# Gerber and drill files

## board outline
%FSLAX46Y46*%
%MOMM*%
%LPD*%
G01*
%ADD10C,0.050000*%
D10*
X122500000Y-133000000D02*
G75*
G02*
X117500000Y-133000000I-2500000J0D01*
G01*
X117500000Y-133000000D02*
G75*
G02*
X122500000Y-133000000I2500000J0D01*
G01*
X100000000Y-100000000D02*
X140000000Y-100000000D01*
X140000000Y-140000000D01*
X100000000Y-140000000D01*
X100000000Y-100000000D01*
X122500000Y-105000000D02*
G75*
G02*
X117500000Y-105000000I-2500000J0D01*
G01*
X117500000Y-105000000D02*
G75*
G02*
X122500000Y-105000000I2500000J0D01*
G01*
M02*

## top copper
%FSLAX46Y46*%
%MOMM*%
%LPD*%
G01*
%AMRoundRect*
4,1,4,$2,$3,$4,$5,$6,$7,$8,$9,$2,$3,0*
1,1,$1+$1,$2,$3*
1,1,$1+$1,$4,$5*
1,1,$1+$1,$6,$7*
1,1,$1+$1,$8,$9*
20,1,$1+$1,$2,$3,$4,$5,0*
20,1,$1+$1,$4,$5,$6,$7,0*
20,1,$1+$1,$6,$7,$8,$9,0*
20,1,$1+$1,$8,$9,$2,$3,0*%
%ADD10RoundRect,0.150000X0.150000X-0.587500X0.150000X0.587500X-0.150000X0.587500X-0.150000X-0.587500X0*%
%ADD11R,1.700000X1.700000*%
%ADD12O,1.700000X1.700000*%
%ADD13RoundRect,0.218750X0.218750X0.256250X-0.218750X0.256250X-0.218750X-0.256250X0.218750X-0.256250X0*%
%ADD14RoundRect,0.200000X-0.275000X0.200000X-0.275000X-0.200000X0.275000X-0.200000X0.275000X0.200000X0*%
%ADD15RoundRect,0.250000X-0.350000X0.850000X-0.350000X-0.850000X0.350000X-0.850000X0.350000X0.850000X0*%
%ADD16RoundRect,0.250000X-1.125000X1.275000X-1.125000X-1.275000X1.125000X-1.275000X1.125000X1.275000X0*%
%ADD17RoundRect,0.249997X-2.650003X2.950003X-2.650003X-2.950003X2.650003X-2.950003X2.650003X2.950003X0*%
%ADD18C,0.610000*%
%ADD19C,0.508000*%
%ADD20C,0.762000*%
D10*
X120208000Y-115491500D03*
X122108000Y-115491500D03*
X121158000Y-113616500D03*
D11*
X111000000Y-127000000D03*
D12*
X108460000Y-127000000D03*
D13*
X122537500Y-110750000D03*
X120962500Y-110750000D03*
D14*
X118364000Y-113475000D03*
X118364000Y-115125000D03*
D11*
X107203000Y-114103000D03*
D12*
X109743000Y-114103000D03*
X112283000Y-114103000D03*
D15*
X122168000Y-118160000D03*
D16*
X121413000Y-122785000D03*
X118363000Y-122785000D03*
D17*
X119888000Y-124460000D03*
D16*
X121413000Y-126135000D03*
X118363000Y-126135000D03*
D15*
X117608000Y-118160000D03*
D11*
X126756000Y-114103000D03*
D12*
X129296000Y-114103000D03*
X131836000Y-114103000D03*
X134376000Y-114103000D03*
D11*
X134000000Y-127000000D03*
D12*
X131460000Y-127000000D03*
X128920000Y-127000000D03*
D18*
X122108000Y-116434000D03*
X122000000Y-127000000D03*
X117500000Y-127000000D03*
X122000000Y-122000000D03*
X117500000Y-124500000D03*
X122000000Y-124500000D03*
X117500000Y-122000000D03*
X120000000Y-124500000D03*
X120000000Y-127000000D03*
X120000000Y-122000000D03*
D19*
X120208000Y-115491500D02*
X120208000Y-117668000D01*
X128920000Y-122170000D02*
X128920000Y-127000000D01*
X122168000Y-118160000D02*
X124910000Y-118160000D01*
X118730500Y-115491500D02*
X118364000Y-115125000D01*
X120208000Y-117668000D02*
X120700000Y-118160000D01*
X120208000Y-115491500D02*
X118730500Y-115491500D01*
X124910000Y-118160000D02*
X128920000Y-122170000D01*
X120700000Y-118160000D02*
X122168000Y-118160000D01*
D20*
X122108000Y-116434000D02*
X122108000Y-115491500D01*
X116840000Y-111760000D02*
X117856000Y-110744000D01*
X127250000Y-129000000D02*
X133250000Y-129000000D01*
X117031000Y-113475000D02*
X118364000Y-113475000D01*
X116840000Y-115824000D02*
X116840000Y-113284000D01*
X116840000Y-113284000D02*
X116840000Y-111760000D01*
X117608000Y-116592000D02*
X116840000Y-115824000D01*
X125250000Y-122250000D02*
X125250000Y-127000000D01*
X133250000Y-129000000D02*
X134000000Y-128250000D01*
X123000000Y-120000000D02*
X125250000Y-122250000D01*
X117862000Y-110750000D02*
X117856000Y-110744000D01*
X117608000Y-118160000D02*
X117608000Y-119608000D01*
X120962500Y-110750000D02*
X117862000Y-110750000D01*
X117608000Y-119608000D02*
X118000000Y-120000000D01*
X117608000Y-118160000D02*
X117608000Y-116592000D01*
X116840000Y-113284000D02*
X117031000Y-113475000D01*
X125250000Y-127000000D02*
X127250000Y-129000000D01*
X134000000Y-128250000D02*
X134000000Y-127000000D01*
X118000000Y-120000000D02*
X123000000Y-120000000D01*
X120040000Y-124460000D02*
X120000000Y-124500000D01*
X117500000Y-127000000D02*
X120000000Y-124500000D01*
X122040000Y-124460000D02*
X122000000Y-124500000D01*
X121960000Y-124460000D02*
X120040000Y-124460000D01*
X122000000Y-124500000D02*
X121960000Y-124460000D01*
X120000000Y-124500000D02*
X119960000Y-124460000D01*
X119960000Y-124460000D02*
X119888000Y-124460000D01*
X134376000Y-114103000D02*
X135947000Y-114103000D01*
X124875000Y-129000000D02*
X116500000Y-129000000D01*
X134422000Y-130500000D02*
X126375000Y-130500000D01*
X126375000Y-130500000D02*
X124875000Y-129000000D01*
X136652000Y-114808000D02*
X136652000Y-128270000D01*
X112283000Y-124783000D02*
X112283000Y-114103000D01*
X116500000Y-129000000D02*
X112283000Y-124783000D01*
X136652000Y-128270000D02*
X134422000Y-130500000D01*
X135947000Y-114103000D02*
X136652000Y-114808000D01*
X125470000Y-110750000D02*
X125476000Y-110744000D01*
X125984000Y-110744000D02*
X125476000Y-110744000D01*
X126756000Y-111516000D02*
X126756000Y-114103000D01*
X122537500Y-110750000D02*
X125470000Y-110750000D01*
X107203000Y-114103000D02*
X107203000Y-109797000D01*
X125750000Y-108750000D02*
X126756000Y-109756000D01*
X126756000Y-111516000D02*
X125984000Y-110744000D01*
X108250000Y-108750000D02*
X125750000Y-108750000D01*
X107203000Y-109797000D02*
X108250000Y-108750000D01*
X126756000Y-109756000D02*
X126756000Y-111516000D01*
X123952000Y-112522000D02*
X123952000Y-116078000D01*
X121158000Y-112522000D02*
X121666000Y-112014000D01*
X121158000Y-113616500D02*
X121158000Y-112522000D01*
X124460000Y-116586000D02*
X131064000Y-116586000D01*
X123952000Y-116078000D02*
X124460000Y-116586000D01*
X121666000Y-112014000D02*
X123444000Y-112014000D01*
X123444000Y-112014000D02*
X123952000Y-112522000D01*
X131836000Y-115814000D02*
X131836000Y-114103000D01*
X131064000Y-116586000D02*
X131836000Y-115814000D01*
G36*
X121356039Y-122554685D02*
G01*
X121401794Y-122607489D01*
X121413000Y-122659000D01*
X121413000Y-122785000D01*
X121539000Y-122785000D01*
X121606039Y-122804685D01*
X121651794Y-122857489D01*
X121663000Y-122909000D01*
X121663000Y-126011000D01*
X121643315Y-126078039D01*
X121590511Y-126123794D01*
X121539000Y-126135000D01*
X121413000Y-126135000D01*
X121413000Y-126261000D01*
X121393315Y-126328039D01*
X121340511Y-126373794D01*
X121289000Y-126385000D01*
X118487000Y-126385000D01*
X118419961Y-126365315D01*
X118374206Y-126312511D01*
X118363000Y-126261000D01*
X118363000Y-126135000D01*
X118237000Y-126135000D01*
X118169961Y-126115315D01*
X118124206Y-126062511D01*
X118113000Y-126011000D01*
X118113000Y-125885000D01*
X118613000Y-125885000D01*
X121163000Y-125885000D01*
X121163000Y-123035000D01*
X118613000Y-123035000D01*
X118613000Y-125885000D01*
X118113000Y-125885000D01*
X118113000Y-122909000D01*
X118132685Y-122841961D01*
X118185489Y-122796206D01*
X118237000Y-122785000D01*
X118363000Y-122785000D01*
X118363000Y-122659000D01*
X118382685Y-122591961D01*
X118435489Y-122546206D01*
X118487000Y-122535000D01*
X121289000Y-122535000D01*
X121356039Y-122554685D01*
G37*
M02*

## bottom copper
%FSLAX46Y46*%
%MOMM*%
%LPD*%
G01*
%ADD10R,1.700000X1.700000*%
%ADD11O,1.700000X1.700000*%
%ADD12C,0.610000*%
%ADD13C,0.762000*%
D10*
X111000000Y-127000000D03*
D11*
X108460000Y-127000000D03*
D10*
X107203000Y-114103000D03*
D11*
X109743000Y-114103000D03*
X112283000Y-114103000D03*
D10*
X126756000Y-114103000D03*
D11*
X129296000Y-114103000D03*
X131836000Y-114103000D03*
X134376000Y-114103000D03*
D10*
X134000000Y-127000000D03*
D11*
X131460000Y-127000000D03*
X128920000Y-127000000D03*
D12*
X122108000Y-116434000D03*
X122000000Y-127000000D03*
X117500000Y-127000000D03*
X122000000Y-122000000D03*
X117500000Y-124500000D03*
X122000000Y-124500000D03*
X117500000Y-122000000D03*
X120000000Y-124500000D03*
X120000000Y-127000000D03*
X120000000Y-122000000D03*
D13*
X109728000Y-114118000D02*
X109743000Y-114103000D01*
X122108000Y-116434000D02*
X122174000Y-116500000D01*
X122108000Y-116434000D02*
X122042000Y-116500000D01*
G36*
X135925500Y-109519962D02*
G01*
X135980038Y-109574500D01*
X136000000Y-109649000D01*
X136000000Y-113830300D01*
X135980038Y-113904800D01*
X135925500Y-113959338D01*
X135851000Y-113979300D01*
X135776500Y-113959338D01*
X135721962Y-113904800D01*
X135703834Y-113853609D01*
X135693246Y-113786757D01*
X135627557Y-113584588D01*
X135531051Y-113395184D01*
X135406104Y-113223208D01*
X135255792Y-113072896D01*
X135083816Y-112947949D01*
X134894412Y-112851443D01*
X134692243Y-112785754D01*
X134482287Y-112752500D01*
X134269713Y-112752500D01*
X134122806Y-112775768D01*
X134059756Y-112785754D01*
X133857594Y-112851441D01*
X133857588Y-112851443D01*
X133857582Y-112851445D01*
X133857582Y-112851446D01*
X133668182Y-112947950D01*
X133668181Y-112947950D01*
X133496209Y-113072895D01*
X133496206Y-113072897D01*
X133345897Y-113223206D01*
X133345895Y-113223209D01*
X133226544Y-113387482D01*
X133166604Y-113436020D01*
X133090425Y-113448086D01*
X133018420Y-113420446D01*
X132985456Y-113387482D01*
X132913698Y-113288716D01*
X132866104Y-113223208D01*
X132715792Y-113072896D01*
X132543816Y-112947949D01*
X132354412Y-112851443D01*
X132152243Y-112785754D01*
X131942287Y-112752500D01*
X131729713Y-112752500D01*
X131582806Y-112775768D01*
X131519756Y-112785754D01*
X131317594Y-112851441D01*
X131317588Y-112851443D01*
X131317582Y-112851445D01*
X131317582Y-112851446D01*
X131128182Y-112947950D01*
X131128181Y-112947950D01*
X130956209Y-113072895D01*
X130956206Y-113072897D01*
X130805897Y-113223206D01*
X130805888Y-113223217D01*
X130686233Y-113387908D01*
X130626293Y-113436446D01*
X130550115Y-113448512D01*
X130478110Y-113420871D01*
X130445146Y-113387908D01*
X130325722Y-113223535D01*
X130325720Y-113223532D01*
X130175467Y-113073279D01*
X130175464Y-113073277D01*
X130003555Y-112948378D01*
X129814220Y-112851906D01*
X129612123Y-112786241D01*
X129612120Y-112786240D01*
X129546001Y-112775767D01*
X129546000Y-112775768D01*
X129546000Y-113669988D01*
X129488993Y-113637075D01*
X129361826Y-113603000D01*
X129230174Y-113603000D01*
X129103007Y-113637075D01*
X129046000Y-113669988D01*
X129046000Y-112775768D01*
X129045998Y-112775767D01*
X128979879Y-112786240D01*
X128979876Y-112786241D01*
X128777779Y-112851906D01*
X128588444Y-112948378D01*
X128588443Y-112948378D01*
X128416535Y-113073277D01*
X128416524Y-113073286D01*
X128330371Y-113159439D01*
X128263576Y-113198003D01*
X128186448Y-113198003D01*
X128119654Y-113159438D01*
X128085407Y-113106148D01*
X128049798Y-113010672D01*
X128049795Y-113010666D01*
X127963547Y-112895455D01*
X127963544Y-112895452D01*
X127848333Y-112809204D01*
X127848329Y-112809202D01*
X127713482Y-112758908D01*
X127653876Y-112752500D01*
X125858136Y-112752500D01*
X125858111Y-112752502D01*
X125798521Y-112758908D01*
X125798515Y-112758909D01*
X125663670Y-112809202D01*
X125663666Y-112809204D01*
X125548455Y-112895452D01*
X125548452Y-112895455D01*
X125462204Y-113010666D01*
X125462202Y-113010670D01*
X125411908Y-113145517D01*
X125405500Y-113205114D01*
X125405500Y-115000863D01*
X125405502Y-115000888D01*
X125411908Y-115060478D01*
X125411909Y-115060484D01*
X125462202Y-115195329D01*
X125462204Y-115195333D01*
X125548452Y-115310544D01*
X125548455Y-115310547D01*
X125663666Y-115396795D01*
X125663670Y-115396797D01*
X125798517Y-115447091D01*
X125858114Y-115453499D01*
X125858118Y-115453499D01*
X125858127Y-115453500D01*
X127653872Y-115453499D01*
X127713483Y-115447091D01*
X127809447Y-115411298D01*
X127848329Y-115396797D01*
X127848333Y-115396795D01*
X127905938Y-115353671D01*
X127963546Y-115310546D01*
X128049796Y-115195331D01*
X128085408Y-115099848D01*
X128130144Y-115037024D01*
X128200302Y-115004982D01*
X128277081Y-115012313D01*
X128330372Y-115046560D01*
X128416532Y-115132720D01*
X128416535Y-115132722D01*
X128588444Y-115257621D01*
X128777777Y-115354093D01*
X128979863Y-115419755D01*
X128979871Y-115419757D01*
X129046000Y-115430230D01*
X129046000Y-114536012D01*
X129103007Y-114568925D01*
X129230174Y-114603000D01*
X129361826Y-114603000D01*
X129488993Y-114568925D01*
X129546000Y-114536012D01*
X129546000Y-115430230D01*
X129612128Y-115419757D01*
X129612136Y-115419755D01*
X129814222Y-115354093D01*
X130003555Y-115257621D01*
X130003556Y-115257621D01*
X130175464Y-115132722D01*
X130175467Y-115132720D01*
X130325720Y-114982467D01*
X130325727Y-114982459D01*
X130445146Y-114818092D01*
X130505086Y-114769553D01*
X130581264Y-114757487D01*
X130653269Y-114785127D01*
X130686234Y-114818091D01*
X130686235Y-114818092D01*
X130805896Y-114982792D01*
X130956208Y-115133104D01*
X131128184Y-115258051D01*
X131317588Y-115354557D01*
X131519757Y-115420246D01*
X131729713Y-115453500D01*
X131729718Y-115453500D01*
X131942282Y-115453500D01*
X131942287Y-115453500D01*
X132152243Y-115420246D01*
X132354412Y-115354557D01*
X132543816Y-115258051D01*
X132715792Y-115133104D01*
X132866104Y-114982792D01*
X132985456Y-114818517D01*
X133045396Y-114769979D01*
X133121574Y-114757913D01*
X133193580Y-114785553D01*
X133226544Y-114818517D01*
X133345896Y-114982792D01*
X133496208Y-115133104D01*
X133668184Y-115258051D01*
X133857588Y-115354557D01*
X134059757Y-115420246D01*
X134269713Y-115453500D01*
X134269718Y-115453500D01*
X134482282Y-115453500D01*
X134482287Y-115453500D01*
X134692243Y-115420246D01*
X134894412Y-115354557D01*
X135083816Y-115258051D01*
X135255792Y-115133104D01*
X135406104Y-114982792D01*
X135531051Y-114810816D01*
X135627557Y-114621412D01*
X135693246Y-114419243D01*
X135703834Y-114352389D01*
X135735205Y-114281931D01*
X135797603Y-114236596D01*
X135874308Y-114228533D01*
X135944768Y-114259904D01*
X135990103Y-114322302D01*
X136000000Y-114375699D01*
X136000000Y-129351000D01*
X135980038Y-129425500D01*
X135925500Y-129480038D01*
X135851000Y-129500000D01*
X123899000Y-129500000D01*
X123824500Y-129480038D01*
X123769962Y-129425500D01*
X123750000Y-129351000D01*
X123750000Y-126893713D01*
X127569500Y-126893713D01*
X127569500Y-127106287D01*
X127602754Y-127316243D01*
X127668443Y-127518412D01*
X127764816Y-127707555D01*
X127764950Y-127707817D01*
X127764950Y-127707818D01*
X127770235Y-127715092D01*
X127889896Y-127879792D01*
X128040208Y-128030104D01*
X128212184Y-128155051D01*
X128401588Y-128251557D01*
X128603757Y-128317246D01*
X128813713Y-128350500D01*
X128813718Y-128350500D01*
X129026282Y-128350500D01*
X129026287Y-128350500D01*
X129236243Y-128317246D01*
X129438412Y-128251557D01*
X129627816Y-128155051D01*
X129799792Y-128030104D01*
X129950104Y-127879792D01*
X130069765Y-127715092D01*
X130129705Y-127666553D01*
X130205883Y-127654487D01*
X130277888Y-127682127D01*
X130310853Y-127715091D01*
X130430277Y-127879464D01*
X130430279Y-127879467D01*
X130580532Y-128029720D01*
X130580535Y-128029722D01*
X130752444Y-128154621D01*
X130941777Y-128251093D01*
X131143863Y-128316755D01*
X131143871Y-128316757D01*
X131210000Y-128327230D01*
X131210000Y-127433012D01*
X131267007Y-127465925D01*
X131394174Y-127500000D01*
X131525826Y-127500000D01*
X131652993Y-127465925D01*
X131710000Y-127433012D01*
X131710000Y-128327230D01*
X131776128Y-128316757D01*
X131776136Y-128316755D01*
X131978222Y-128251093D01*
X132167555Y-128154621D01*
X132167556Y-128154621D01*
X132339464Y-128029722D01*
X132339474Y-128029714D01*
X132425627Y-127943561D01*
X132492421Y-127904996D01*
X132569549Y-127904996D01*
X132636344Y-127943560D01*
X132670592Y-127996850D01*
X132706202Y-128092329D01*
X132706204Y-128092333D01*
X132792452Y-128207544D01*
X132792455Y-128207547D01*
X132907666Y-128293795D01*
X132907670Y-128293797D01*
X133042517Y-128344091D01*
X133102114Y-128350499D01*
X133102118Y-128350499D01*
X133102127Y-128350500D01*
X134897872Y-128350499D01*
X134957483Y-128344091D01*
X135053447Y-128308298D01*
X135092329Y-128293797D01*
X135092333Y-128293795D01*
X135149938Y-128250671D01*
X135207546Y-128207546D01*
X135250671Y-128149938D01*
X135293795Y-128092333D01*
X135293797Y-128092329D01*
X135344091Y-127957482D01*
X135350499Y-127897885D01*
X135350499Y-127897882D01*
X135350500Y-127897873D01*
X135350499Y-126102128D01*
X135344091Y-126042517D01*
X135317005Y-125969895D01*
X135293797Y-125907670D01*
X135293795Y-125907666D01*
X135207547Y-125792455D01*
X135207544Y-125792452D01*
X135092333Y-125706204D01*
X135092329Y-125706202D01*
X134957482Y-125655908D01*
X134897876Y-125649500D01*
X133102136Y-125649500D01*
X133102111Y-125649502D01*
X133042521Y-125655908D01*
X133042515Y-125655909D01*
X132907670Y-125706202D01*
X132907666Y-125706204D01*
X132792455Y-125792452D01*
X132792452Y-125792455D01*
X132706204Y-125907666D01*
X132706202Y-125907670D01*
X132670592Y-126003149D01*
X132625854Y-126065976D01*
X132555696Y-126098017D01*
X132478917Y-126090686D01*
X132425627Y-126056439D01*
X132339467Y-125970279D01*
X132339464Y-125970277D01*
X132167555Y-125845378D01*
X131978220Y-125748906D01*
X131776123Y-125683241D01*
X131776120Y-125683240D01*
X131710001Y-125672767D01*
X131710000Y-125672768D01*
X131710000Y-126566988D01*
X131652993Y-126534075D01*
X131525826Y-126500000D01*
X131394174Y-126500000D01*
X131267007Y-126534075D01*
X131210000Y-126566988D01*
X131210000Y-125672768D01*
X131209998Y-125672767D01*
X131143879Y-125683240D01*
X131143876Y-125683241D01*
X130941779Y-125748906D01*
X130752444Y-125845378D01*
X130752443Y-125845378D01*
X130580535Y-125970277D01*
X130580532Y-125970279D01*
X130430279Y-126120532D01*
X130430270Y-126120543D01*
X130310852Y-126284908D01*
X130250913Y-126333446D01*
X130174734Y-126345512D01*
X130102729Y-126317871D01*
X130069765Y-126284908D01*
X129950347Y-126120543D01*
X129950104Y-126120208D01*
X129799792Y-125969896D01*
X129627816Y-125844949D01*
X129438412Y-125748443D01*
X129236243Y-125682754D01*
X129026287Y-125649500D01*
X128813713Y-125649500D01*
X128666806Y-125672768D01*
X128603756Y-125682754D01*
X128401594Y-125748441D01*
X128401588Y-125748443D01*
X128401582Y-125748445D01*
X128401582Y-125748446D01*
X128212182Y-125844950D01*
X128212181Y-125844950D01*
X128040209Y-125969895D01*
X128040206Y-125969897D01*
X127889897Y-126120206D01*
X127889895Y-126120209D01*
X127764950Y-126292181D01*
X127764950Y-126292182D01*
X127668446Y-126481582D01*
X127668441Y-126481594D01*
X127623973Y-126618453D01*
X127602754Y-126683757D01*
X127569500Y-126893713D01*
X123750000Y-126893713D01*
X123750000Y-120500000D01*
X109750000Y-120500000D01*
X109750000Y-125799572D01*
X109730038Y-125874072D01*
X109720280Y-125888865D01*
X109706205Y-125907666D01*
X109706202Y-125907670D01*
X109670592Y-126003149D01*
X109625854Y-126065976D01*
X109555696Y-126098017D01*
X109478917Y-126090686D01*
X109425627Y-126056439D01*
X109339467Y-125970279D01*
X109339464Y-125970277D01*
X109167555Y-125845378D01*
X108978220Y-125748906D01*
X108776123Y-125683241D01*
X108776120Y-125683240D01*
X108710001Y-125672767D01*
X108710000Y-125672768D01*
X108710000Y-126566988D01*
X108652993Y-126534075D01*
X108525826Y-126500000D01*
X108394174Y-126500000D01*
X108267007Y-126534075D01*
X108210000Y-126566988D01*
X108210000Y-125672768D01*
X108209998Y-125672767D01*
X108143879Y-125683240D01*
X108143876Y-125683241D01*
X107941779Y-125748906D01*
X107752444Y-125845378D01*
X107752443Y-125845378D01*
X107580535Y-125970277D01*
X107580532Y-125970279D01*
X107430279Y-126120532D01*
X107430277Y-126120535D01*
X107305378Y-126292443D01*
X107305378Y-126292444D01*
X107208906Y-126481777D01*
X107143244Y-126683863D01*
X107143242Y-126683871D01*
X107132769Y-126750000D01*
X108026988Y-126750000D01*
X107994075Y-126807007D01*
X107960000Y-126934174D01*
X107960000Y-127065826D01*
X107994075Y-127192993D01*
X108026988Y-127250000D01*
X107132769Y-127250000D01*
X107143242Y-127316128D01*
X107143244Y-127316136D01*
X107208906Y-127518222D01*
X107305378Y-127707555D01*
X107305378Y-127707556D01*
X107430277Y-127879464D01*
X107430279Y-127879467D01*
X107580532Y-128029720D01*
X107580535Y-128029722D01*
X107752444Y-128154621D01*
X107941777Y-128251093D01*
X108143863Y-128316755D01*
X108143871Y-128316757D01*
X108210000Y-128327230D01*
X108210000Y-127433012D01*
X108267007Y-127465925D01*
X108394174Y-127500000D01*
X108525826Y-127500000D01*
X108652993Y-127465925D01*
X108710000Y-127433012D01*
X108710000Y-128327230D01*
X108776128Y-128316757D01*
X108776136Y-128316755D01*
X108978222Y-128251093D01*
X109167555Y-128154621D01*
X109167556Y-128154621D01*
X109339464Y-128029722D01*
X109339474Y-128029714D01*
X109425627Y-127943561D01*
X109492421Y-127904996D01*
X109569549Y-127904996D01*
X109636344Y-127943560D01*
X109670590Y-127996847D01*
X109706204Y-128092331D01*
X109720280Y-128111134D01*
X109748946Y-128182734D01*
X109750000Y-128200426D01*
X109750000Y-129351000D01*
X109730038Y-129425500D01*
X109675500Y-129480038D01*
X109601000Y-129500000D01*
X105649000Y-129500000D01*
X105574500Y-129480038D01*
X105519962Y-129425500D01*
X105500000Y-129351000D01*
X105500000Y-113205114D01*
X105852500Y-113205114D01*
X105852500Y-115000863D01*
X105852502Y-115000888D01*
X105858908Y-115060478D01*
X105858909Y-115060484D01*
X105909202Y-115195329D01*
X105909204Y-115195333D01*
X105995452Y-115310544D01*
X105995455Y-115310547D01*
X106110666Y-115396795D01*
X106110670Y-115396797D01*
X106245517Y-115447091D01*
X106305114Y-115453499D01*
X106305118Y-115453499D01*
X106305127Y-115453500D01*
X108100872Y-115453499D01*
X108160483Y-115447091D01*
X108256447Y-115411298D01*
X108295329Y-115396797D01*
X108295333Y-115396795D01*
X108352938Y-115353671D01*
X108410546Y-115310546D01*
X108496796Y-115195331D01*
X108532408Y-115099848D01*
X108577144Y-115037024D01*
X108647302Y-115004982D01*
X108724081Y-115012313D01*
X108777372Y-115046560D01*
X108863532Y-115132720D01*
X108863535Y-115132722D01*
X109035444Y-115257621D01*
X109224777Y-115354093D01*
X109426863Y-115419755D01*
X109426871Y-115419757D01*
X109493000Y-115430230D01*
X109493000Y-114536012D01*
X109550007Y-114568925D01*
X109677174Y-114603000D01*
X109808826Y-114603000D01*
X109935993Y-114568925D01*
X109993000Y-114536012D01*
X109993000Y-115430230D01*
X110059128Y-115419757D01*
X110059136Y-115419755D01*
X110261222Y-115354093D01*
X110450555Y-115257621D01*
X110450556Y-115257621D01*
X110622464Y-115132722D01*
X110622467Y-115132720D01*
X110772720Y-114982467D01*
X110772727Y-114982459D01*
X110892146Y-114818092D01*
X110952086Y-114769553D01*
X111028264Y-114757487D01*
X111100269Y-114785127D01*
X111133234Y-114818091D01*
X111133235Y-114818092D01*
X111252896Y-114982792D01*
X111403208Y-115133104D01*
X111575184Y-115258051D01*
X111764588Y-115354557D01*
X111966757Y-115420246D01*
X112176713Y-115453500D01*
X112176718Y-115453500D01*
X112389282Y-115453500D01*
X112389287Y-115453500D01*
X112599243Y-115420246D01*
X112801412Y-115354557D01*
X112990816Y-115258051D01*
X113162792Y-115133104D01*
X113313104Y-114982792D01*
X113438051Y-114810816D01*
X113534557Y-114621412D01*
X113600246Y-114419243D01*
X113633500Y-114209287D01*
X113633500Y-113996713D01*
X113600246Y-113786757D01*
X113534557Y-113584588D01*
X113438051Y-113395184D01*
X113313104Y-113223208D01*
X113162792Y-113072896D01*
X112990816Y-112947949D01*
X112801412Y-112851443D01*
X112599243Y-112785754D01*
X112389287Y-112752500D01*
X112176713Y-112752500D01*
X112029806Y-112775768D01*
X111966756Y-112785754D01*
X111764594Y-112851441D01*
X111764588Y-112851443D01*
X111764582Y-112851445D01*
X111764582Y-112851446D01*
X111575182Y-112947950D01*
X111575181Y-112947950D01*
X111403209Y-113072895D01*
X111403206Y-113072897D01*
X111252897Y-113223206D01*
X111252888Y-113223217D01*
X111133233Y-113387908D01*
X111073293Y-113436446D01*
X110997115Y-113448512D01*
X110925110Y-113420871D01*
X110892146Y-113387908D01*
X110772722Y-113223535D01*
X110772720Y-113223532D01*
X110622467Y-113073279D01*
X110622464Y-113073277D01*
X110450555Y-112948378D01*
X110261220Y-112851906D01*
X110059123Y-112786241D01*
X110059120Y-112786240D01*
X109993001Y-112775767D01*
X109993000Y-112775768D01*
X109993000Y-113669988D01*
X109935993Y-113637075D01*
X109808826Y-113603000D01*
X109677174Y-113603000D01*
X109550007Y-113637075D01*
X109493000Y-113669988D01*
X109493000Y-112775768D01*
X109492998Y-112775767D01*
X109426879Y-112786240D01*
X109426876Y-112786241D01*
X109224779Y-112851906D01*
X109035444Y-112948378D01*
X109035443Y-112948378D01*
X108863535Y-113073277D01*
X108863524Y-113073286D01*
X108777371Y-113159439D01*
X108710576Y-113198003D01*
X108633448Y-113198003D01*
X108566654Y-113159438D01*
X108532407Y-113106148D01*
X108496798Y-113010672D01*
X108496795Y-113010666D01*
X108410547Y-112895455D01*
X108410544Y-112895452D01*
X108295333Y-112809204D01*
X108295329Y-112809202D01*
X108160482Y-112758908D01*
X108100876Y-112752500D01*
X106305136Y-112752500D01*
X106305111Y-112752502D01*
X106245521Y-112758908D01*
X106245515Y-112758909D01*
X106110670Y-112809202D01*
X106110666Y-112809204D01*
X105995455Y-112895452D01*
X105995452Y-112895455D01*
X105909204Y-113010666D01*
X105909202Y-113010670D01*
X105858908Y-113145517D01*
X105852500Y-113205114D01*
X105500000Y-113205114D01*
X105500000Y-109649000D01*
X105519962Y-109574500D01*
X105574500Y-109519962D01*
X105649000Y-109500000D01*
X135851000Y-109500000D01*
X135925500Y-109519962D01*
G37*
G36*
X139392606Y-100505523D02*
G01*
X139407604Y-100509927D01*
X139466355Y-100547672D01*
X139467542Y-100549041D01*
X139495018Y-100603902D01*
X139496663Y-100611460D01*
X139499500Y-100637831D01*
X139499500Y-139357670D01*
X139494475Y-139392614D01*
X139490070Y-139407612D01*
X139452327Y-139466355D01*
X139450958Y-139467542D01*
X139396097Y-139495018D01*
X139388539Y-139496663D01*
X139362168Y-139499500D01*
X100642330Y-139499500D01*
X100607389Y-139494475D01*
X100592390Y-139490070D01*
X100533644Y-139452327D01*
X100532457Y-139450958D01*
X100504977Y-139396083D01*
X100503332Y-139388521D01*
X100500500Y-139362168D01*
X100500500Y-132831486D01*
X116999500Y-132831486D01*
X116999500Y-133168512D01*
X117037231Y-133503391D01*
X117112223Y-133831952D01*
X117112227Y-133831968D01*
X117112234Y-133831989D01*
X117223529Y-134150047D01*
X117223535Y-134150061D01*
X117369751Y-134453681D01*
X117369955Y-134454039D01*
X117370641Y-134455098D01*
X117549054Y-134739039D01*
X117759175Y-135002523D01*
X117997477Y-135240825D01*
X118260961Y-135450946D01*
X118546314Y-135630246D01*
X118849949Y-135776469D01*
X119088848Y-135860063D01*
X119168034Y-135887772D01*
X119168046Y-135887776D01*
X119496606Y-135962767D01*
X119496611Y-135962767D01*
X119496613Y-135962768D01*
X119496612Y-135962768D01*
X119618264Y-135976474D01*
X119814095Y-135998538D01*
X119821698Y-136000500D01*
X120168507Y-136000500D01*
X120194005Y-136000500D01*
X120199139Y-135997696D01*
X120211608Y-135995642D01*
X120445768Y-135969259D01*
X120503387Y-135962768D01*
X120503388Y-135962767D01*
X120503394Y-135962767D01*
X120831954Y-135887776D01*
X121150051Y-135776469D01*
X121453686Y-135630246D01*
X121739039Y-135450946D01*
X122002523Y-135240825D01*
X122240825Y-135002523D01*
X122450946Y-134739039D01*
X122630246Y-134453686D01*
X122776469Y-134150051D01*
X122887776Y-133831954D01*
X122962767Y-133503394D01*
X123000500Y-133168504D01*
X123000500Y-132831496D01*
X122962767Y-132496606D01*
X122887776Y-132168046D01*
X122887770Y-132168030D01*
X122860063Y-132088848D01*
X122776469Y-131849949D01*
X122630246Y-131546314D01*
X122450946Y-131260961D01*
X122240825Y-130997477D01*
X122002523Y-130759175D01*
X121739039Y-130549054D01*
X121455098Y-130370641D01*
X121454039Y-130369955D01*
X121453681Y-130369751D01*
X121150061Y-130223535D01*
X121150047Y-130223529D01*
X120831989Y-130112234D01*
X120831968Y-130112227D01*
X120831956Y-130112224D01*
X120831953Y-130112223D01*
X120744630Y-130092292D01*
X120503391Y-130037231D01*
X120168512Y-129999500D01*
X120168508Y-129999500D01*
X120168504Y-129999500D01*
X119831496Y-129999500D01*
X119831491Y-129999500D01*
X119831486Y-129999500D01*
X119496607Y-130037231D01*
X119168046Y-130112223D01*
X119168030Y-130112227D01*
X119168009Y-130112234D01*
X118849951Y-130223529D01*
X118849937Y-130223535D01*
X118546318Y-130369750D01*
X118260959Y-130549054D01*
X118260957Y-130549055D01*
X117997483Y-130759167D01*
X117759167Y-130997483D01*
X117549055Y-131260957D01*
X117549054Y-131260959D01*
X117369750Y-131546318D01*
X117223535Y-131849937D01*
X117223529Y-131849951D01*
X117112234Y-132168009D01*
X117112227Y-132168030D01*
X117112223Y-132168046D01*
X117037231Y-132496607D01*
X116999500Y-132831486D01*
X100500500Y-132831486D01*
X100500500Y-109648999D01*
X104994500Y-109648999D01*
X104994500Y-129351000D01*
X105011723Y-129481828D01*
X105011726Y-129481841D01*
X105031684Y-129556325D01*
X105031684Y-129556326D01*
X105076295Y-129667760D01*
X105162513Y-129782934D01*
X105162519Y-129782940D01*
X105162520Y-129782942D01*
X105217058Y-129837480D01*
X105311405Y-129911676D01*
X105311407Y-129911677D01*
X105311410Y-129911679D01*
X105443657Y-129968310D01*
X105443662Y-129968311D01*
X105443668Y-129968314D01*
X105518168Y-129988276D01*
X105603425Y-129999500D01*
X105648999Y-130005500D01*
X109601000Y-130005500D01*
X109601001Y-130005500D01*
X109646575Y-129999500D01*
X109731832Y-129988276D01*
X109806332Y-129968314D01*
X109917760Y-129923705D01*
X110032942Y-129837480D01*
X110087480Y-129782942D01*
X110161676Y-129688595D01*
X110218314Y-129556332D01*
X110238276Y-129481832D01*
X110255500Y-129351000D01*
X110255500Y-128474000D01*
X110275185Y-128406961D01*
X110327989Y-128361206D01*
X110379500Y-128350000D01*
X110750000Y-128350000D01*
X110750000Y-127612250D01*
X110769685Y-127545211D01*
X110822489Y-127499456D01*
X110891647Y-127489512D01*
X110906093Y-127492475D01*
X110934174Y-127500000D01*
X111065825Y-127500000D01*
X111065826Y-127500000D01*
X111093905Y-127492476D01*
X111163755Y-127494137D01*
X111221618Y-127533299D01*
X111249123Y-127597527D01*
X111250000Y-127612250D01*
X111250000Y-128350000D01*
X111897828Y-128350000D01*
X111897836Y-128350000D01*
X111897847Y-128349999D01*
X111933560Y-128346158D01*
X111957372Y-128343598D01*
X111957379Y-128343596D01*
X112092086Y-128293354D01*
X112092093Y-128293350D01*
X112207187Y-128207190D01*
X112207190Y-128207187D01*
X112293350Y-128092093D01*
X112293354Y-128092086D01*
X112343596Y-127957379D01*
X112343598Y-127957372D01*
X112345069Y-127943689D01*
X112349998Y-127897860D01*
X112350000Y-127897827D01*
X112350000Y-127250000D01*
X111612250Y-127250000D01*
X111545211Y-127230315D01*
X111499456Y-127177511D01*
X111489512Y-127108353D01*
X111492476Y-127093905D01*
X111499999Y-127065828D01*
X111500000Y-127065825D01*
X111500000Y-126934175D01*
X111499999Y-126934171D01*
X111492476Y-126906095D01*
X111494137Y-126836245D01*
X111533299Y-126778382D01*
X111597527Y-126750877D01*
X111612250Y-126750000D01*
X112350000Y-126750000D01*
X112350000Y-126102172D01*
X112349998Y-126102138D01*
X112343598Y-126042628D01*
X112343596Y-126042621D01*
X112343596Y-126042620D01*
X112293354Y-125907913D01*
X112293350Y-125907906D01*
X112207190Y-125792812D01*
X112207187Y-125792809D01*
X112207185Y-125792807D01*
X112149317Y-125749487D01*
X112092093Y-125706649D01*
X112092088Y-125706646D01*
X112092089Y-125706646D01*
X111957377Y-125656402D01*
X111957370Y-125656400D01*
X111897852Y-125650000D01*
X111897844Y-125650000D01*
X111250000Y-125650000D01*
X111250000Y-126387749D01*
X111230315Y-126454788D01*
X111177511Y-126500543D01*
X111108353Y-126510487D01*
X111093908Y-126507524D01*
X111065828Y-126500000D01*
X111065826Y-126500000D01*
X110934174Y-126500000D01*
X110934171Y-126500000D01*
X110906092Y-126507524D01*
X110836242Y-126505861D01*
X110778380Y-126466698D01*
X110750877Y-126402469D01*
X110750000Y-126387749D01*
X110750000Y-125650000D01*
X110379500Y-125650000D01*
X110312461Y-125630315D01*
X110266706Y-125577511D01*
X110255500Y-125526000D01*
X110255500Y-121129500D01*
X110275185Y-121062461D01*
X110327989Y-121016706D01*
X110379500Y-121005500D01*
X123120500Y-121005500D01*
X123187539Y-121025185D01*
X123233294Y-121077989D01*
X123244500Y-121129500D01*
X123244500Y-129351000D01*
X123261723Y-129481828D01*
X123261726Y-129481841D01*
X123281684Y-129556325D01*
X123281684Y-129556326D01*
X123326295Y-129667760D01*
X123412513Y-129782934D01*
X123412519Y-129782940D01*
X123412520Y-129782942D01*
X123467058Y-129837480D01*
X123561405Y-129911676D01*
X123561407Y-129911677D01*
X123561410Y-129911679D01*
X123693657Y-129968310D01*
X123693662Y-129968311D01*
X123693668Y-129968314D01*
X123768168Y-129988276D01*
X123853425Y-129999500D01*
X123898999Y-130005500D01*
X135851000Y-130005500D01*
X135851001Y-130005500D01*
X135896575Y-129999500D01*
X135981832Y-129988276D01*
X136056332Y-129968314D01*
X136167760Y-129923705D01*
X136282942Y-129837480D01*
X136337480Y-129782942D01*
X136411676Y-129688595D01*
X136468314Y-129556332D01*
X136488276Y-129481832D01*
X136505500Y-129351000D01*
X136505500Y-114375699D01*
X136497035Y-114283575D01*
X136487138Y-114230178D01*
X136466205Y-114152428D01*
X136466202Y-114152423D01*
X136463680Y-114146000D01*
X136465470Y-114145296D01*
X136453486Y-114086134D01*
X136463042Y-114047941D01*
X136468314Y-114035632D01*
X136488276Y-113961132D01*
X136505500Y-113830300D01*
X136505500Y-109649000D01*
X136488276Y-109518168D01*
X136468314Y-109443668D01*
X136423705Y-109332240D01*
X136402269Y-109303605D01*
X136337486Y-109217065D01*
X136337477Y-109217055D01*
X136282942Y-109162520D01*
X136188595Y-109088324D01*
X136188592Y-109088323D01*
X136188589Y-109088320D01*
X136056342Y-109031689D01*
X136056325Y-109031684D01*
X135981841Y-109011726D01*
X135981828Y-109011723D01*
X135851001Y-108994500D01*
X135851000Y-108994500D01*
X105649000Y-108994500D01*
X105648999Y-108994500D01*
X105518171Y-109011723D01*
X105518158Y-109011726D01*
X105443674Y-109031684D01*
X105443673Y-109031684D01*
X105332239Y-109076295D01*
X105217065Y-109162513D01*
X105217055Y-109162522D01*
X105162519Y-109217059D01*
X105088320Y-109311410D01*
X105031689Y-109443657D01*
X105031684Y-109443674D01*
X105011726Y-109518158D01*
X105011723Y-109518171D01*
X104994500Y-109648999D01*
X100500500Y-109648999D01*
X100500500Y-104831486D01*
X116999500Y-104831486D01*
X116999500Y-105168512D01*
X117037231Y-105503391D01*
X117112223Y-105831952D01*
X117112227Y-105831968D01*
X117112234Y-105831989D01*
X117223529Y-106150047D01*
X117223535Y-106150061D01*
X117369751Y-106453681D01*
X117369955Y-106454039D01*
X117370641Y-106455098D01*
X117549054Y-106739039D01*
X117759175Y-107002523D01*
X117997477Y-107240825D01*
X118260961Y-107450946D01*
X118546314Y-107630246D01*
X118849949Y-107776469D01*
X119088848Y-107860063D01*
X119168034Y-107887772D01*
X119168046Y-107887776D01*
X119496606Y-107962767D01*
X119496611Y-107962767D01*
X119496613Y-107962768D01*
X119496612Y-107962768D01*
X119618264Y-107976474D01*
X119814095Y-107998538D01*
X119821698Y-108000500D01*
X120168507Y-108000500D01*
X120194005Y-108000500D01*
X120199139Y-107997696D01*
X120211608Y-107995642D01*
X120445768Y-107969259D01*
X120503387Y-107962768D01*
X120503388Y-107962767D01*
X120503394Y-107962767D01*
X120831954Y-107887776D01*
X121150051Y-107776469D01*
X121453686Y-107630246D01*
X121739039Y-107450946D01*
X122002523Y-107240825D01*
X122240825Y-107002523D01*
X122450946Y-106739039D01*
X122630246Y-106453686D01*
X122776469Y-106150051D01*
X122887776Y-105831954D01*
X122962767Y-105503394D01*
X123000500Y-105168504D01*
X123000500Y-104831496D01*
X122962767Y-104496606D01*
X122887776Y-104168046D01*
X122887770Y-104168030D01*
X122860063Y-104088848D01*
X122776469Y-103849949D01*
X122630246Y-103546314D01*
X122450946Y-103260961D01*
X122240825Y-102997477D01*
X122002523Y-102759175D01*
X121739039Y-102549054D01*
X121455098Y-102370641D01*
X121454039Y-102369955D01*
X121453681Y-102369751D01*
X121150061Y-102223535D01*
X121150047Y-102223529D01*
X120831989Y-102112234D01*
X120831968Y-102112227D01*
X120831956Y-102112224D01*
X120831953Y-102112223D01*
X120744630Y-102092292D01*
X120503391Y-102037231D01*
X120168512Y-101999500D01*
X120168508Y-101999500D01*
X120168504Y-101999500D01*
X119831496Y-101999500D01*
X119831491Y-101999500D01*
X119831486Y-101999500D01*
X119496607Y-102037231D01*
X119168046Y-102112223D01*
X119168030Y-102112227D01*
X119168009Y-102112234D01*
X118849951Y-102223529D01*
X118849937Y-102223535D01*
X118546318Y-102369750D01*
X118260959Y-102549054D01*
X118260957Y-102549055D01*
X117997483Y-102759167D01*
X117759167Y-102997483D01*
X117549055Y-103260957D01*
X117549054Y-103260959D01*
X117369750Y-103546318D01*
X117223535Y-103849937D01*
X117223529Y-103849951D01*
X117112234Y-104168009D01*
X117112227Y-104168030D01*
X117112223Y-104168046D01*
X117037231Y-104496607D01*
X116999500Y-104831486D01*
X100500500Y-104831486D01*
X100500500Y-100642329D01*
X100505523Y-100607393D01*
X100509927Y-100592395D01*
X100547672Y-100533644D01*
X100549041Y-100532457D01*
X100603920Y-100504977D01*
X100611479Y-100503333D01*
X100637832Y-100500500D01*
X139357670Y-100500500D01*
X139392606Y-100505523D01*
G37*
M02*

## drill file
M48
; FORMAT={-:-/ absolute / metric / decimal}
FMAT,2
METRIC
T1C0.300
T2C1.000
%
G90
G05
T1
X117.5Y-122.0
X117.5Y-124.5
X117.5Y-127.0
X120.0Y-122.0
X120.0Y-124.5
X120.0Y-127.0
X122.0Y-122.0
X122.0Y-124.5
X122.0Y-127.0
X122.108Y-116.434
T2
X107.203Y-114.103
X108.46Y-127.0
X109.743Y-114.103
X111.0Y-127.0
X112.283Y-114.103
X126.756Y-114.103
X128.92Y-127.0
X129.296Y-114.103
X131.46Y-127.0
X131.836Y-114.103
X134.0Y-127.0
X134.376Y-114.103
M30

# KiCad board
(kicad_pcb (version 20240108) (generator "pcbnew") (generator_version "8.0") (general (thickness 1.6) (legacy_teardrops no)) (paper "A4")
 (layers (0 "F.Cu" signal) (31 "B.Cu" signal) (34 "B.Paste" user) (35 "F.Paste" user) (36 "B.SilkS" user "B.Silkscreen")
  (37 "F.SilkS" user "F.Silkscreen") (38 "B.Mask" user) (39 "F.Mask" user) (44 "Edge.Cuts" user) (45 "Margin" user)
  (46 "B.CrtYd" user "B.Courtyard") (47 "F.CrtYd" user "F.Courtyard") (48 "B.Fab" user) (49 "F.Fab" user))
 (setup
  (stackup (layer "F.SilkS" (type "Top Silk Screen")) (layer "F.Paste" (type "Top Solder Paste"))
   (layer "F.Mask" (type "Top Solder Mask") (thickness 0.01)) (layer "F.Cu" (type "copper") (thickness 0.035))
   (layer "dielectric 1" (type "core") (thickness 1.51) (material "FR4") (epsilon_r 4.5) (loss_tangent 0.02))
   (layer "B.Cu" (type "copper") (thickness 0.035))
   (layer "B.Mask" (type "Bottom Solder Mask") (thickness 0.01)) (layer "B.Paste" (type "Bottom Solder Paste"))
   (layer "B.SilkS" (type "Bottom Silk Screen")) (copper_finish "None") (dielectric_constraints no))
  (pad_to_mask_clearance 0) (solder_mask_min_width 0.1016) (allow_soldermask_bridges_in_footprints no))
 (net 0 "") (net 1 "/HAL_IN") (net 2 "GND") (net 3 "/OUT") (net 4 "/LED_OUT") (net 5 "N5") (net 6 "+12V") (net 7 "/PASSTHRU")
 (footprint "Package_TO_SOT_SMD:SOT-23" (layer "F.Cu") (at 121.158 114.554 90)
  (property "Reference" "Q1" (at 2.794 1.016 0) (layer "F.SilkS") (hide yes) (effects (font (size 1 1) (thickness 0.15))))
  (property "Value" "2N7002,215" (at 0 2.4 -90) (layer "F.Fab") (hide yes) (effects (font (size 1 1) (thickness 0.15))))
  (pad "1" smd roundrect (at -0.9375 -0.95 90) (size 1.475 0.6) (layers "F.Cu" "F.Paste" "F.Mask") (roundrect_rratio 0.25) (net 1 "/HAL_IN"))
  (pad "2" smd roundrect (at -0.9375 0.95 90) (size 1.475 0.6) (layers "F.Cu" "F.Paste" "F.Mask") (roundrect_rratio 0.25) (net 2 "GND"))
  (pad "3" smd roundrect (at 0.9375 0 90) (size 1.475 0.6) (layers "F.Cu" "F.Paste" "F.Mask") (roundrect_rratio 0.25) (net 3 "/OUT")))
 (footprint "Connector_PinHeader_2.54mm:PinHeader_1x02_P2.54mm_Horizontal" (layer "F.Cu") (at 111 127 -90)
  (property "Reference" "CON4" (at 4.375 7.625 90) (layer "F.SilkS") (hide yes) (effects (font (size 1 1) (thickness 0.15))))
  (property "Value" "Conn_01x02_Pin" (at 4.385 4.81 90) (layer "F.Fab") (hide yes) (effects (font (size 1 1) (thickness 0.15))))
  (pad "1" thru_hole rect (at 0 0 270) (size 1.7 1.7) (drill 1) (layers "*.Cu" "*.Mask") (remove_unused_layers no) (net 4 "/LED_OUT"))
  (pad "2" thru_hole oval (at 0 2.54 270) (size 1.7 1.7) (drill 1) (layers "*.Cu" "*.Mask") (remove_unused_layers no) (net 2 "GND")))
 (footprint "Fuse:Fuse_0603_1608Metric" (layer "F.Cu") (at 121.75 110.75 180)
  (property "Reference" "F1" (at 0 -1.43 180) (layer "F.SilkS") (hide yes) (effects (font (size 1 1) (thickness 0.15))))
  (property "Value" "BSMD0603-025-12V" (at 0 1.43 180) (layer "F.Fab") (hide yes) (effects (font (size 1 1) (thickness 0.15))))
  (pad "1" smd roundrect (at -0.7875 0 180) (size 0.875 0.95) (layers "F.Cu" "F.Paste" "F.Mask") (roundrect_rratio 0.25) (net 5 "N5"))
  (pad "2" smd roundrect (at 0.7875 0 180) (size 0.875 0.95) (layers "F.Cu" "F.Paste" "F.Mask") (roundrect_rratio 0.25) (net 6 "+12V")))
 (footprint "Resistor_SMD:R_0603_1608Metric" (layer "F.Cu") (at 118.364 114.3 -90)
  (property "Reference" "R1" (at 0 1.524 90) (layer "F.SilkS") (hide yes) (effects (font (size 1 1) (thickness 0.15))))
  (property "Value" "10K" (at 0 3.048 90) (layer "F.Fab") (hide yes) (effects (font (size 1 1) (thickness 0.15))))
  (pad "1" smd roundrect (at -0.825 0 270) (size 0.8 0.95) (layers "F.Cu" "F.Paste" "F.Mask") (roundrect_rratio 0.25) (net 6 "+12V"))
  (pad "2" smd roundrect (at 0.825 0 270) (size 0.8 0.95) (layers "F.Cu" "F.Paste" "F.Mask") (roundrect_rratio 0.25) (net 1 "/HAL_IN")))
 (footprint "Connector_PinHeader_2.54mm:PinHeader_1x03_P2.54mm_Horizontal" (layer "F.Cu") (at 107.203 114.103 90)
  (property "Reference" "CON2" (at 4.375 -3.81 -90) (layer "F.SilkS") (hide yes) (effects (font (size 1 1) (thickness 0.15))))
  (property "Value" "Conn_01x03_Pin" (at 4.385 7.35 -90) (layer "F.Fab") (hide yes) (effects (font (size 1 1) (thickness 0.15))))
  (pad "1" thru_hole rect (at 0 0 90) (size 1.7 1.7) (drill 1) (layers "*.Cu" "*.Mask") (remove_unused_layers no) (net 5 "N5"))
  (pad "2" thru_hole oval (at 0 2.54 90) (size 1.7 1.7) (drill 1) (layers "*.Cu" "*.Mask") (remove_unused_layers no) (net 2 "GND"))
  (pad "3" thru_hole oval (at 0 5.08 90) (size 1.7 1.7) (drill 1) (layers "*.Cu" "*.Mask") (remove_unused_layers no) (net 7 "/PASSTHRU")))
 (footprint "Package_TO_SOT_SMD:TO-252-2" (layer "F.Cu") (at 119.888 123.2 -90)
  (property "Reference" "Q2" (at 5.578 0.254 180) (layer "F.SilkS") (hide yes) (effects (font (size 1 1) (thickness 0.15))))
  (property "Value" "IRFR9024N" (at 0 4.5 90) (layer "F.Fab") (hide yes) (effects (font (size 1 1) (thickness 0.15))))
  (pad "1" smd roundrect (at -5.04 -2.28 270) (size 2.2 1.2) (layers "F.Cu" "F.Paste" "F.Mask") (roundrect_rratio 0.208333)
   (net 1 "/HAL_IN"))
  (pad "2" smd roundrect (at -0.415 -1.525 270) (size 3.05 2.75) (layers "F.Cu" "F.Paste") (roundrect_rratio 0.090909) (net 4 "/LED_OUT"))
  (pad "2" smd roundrect (at -0.415 1.525 270) (size 3.05 2.75) (layers "F.Cu" "F.Paste") (roundrect_rratio 0.090909) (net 4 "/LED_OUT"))
  (pad "2" smd roundrect (at 1.26 0 270) (size 6.4 5.8) (layers "F.Cu" "F.Mask") (roundrect_rratio 0.043103) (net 4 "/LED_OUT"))
  (pad "2" smd roundrect (at 2.935 -1.525 270) (size 3.05 2.75) (layers "F.Cu" "F.Paste") (roundrect_rratio 0.090909) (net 4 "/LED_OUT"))
  (pad "2" smd roundrect (at 2.935 1.525 270) (size 3.05 2.75) (layers "F.Cu" "F.Paste") (roundrect_rratio 0.090909) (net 4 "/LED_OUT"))
  (pad "3" smd roundrect (at -5.04 2.28 270) (size 2.2 1.2) (layers "F.Cu" "F.Paste" "F.Mask") (roundrect_rratio 0.208333) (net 6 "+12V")))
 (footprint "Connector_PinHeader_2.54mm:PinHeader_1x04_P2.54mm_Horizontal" (layer "F.Cu") (at 126.756 114.103 90)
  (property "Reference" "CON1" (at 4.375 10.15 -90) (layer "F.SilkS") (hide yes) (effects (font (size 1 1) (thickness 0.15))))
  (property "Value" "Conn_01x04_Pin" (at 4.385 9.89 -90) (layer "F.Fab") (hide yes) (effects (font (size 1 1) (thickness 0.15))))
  (pad "1" thru_hole rect (at 0 0 90) (size 1.7 1.7) (drill 1) (layers "*.Cu" "*.Mask") (remove_unused_layers no) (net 5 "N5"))
  (pad "2" thru_hole oval (at 0 2.54 90) (size 1.7 1.7) (drill 1) (layers "*.Cu" "*.Mask") (remove_unused_layers no) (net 2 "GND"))
  (pad "3" thru_hole oval (at 0 5.08 90) (size 1.7 1.7) (drill 1) (layers "*.Cu" "*.Mask") (remove_unused_layers no) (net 3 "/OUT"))
  (pad "4" thru_hole oval (at 0 7.62 90) (size 1.7 1.7) (drill 1) (layers "*.Cu" "*.Mask") (remove_unused_layers no) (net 7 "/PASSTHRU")))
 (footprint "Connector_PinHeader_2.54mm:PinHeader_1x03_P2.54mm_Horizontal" (layer "F.Cu") (at 134 127 -90)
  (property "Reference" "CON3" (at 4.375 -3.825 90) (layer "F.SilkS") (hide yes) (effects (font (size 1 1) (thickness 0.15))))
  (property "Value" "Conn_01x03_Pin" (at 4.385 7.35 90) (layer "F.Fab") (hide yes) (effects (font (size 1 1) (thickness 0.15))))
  (pad "1" thru_hole rect (at 0 0 270) (size 1.7 1.7) (drill 1) (layers "*.Cu" "*.Mask") (remove_unused_layers no) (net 6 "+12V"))
  (pad "2" thru_hole oval (at 0 2.54 270) (size 1.7 1.7) (drill 1) (layers "*.Cu" "*.Mask") (remove_unused_layers no) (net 2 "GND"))
  (pad "3" thru_hole oval (at 0 5.08 270) (size 1.7 1.7) (drill 1) (layers "*.Cu" "*.Mask") (remove_unused_layers no) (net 1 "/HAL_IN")))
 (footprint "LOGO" (layer "F.Cu") (at 124.968 133.096)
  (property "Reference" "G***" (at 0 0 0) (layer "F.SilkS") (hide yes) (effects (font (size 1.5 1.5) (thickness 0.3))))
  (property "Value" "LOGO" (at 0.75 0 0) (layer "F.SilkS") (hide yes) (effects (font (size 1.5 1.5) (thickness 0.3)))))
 (gr_circle (center 120 133) (end 122.5 133) (stroke (width 0.05) (type default)) (fill none) (layer "Edge.Cuts"))
 (gr_rect (start 100 100) (end 140 140) (stroke (width 0.05) (type default)) (fill none) (layer "Edge.Cuts"))
 (gr_circle (center 120 105) (end 122.5 105) (stroke (width 0.05) (type default)) (fill none) (layer "Edge.Cuts"))
 (segment (start 120.208 115.4915) (end 120.208 117.668) (width 0.508) (layer "F.Cu") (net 1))
 (segment (start 128.92 122.17) (end 128.92 127) (width 0.508) (layer "F.Cu") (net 1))
 (segment (start 122.168 118.16) (end 124.91 118.16) (width 0.508) (layer "F.Cu") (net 1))
 (segment (start 118.7305 115.4915) (end 118.364 115.125) (width 0.508) (layer "F.Cu") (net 1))
 (segment (start 120.208 117.668) (end 120.7 118.16) (width 0.508) (layer "F.Cu") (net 1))
 (segment (start 120.208 115.4915) (end 118.7305 115.4915) (width 0.508) (layer "F.Cu") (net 1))
 (segment (start 124.91 118.16) (end 128.92 122.17) (width 0.508) (layer "F.Cu") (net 1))
 (segment (start 120.7 118.16) (end 122.168 118.16) (width 0.508) (layer "F.Cu") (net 1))
 (segment (start 122.108 116.434) (end 122.108 115.4915) (width 0.762) (layer "F.Cu") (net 2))
 (via (at 122.108 116.434) (size 0.61) (drill 0.3) (layers "F.Cu" "B.Cu") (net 2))
 (segment (start 109.728 114.118) (end 109.743 114.103) (width 0.762) (layer "B.Cu") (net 2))
 (segment (start 122.108 116.434) (end 122.174 116.5) (width 0.762) (layer "B.Cu") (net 2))
 (segment (start 122.108 116.434) (end 122.042 116.5) (width 0.762) (layer "B.Cu") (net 2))
 (segment (start 116.84 111.76) (end 117.856 110.744) (width 0.762) (layer "F.Cu") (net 6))
 (segment (start 127.25 129) (end 133.25 129) (width 0.762) (layer "F.Cu") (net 6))
 (segment (start 117.031 113.475) (end 118.364 113.475) (width 0.762) (layer "F.Cu") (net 6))
 (segment (start 116.84 115.824) (end 116.84 113.284) (width 0.762) (layer "F.Cu") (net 6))
 (segment (start 116.84 113.284) (end 116.84 111.76) (width 0.762) (layer "F.Cu") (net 6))
 (segment (start 117.608 116.592) (end 116.84 115.824) (width 0.762) (layer "F.Cu") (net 6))
 (segment (start 125.25 122.25) (end 125.25 127) (width 0.762) (layer "F.Cu") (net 6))
 (segment (start 133.25 129) (end 134 128.25) (width 0.762) (layer "F.Cu") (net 6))
 (segment (start 123 120) (end 125.25 122.25) (width 0.762) (layer "F.Cu") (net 6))
 (segment (start 117.862 110.75) (end 117.856 110.744) (width 0.762) (layer "F.Cu") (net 6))
 (segment (start 117.608 118.16) (end 117.608 119.608) (width 0.762) (layer "F.Cu") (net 6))
 (segment (start 120.9625 110.75) (end 117.862 110.75) (width 0.762) (layer "F.Cu") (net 6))
 (segment (start 117.608 119.608) (end 118 120) (width 0.762) (layer "F.Cu") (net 6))
 (segment (start 117.608 118.16) (end 117.608 116.592) (width 0.762) (layer "F.Cu") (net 6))
 (segment (start 116.84 113.284) (end 117.031 113.475) (width 0.762) (layer "F.Cu") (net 6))
 (segment (start 125.25 127) (end 127.25 129) (width 0.762) (layer "F.Cu") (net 6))
 (segment (start 134 128.25) (end 134 127) (width 0.762) (layer "F.Cu") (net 6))
 (segment (start 118 120) (end 123 120) (width 0.762) (layer "F.Cu") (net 6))
 (segment (start 120.04 124.46) (end 120 124.5) (width 0.762) (layer "F.Cu") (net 4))
 (segment (start 117.5 127) (end 120 124.5) (width 0.762) (layer "F.Cu") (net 4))
 (segment (start 122.04 124.46) (end 122 124.5) (width 0.762) (layer "F.Cu") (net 4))
 (segment (start 121.96 124.46) (end 120.04 124.46) (width 0.762) (layer "F.Cu") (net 4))
 (segment (start 122 124.5) (end 121.96 124.46) (width 0.762) (layer "F.Cu") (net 4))
 (segment (start 120 124.5) (end 119.96 124.46) (width 0.762) (layer "F.Cu") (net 4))
 (segment (start 119.96 124.46) (end 119.888 124.46) (width 0.762) (layer "F.Cu") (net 4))
 (via (at 122 127) (size 0.61) (drill 0.3) (layers "F.Cu" "B.Cu") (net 4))
 (via (at 117.5 127) (size 0.61) (drill 0.3) (layers "F.Cu" "B.Cu") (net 4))
 (via (at 122 122) (size 0.61) (drill 0.3) (layers "F.Cu" "B.Cu") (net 4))
 (via (at 117.5 124.5) (size 0.61) (drill 0.3) (layers "F.Cu" "B.Cu") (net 4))
 (via (at 122 124.5) (size 0.61) (drill 0.3) (layers "F.Cu" "B.Cu") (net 4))
 (via (at 117.5 122) (size 0.61) (drill 0.3) (layers "F.Cu" "B.Cu") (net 4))
 (via (at 120 124.5) (size 0.61) (drill 0.3) (layers "F.Cu" "B.Cu") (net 4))
 (via (at 120 127) (size 0.61) (drill 0.3) (layers "F.Cu" "B.Cu") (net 4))
 (via (at 120 122) (size 0.61) (drill 0.3) (layers "F.Cu" "B.Cu") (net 4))
 (segment (start 134.376 114.103) (end 135.947 114.103) (width 0.762) (layer "F.Cu") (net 7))
 (segment (start 124.875 129) (end 116.5 129) (width 0.762) (layer "F.Cu") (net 7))
 (segment (start 134.422 130.5) (end 126.375 130.5) (width 0.762) (layer "F.Cu") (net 7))
 (segment (start 126.375 130.5) (end 124.875 129) (width 0.762) (layer "F.Cu") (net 7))
 (segment (start 136.652 114.808) (end 136.652 128.27) (width 0.762) (layer "F.Cu") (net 7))
 (segment (start 112.283 124.783) (end 112.283 114.103) (width 0.762) (layer "F.Cu") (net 7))
 (segment (start 116.5 129) (end 112.283 124.783) (width 0.762) (layer "F.Cu") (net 7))
 (segment (start 136.652 128.27) (end 134.422 130.5) (width 0.762) (layer "F.Cu") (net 7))
 (segment (start 135.947 114.103) (end 136.652 114.808) (width 0.762) (layer "F.Cu") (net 7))
 (segment (start 125.47 110.75) (end 125.476 110.744) (width 0.762) (layer "F.Cu") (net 5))
 (segment (start 125.984 110.744) (end 125.476 110.744) (width 0.762) (layer "F.Cu") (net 5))
 (segment (start 126.756 111.516) (end 126.756 114.103) (width 0.762) (layer "F.Cu") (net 5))
 (segment (start 122.5375 110.75) (end 125.47 110.75) (width 0.762) (layer "F.Cu") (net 5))
 (segment (start 107.203 114.103) (end 107.203 109.797) (width 0.762) (layer "F.Cu") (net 5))
 (segment (start 125.75 108.75) (end 126.756 109.756) (width 0.762) (layer "F.Cu") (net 5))
 (segment (start 126.756 111.516) (end 125.984 110.744) (width 0.762) (layer "F.Cu") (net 5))
 (segment (start 108.25 108.75) (end 125.75 108.75) (width 0.762) (layer "F.Cu") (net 5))
 (segment (start 107.203 109.797) (end 108.25 108.75) (width 0.762) (layer "F.Cu") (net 5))
 (segment (start 126.756 109.756) (end 126.756 111.516) (width 0.762) (layer "F.Cu") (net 5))
 (segment (start 123.952 112.522) (end 123.952 116.078) (width 0.762) (layer "F.Cu") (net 3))
 (segment (start 121.158 112.522) (end 121.666 112.014) (width 0.762) (layer "F.Cu") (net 3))
 (segment (start 121.158 113.6165) (end 121.158 112.522) (width 0.762) (layer "F.Cu") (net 3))
 (segment (start 124.46 116.586) (end 131.064 116.586) (width 0.762) (layer "F.Cu") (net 3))
 (segment (start 123.952 116.078) (end 124.46 116.586) (width 0.762) (layer "F.Cu") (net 3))
 (segment (start 121.666 112.014) (end 123.444 112.014) (width 0.762) (layer "F.Cu") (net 3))
 (segment (start 123.444 112.014) (end 123.952 112.522) (width 0.762) (layer "F.Cu") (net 3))
 (segment (start 131.836 115.814) (end 131.836 114.103) (width 0.762) (layer "F.Cu") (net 3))
 (segment (start 131.064 116.586) (end 131.836 115.814) (width 0.762) (layer "F.Cu") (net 3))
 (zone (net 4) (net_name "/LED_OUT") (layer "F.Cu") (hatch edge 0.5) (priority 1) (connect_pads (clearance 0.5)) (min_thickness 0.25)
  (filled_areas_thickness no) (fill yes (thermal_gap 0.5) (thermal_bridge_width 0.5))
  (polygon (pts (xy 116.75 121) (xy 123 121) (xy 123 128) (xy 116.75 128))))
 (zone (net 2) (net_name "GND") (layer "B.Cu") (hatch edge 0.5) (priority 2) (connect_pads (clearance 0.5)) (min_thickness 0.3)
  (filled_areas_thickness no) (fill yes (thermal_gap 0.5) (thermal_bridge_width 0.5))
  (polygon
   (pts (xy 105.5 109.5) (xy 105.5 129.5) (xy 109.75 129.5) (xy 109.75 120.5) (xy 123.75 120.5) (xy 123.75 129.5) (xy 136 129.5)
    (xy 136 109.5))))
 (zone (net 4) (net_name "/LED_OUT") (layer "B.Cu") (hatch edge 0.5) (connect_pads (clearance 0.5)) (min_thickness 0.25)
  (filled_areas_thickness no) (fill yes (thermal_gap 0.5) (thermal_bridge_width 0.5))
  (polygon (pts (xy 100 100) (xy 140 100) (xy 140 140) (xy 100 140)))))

